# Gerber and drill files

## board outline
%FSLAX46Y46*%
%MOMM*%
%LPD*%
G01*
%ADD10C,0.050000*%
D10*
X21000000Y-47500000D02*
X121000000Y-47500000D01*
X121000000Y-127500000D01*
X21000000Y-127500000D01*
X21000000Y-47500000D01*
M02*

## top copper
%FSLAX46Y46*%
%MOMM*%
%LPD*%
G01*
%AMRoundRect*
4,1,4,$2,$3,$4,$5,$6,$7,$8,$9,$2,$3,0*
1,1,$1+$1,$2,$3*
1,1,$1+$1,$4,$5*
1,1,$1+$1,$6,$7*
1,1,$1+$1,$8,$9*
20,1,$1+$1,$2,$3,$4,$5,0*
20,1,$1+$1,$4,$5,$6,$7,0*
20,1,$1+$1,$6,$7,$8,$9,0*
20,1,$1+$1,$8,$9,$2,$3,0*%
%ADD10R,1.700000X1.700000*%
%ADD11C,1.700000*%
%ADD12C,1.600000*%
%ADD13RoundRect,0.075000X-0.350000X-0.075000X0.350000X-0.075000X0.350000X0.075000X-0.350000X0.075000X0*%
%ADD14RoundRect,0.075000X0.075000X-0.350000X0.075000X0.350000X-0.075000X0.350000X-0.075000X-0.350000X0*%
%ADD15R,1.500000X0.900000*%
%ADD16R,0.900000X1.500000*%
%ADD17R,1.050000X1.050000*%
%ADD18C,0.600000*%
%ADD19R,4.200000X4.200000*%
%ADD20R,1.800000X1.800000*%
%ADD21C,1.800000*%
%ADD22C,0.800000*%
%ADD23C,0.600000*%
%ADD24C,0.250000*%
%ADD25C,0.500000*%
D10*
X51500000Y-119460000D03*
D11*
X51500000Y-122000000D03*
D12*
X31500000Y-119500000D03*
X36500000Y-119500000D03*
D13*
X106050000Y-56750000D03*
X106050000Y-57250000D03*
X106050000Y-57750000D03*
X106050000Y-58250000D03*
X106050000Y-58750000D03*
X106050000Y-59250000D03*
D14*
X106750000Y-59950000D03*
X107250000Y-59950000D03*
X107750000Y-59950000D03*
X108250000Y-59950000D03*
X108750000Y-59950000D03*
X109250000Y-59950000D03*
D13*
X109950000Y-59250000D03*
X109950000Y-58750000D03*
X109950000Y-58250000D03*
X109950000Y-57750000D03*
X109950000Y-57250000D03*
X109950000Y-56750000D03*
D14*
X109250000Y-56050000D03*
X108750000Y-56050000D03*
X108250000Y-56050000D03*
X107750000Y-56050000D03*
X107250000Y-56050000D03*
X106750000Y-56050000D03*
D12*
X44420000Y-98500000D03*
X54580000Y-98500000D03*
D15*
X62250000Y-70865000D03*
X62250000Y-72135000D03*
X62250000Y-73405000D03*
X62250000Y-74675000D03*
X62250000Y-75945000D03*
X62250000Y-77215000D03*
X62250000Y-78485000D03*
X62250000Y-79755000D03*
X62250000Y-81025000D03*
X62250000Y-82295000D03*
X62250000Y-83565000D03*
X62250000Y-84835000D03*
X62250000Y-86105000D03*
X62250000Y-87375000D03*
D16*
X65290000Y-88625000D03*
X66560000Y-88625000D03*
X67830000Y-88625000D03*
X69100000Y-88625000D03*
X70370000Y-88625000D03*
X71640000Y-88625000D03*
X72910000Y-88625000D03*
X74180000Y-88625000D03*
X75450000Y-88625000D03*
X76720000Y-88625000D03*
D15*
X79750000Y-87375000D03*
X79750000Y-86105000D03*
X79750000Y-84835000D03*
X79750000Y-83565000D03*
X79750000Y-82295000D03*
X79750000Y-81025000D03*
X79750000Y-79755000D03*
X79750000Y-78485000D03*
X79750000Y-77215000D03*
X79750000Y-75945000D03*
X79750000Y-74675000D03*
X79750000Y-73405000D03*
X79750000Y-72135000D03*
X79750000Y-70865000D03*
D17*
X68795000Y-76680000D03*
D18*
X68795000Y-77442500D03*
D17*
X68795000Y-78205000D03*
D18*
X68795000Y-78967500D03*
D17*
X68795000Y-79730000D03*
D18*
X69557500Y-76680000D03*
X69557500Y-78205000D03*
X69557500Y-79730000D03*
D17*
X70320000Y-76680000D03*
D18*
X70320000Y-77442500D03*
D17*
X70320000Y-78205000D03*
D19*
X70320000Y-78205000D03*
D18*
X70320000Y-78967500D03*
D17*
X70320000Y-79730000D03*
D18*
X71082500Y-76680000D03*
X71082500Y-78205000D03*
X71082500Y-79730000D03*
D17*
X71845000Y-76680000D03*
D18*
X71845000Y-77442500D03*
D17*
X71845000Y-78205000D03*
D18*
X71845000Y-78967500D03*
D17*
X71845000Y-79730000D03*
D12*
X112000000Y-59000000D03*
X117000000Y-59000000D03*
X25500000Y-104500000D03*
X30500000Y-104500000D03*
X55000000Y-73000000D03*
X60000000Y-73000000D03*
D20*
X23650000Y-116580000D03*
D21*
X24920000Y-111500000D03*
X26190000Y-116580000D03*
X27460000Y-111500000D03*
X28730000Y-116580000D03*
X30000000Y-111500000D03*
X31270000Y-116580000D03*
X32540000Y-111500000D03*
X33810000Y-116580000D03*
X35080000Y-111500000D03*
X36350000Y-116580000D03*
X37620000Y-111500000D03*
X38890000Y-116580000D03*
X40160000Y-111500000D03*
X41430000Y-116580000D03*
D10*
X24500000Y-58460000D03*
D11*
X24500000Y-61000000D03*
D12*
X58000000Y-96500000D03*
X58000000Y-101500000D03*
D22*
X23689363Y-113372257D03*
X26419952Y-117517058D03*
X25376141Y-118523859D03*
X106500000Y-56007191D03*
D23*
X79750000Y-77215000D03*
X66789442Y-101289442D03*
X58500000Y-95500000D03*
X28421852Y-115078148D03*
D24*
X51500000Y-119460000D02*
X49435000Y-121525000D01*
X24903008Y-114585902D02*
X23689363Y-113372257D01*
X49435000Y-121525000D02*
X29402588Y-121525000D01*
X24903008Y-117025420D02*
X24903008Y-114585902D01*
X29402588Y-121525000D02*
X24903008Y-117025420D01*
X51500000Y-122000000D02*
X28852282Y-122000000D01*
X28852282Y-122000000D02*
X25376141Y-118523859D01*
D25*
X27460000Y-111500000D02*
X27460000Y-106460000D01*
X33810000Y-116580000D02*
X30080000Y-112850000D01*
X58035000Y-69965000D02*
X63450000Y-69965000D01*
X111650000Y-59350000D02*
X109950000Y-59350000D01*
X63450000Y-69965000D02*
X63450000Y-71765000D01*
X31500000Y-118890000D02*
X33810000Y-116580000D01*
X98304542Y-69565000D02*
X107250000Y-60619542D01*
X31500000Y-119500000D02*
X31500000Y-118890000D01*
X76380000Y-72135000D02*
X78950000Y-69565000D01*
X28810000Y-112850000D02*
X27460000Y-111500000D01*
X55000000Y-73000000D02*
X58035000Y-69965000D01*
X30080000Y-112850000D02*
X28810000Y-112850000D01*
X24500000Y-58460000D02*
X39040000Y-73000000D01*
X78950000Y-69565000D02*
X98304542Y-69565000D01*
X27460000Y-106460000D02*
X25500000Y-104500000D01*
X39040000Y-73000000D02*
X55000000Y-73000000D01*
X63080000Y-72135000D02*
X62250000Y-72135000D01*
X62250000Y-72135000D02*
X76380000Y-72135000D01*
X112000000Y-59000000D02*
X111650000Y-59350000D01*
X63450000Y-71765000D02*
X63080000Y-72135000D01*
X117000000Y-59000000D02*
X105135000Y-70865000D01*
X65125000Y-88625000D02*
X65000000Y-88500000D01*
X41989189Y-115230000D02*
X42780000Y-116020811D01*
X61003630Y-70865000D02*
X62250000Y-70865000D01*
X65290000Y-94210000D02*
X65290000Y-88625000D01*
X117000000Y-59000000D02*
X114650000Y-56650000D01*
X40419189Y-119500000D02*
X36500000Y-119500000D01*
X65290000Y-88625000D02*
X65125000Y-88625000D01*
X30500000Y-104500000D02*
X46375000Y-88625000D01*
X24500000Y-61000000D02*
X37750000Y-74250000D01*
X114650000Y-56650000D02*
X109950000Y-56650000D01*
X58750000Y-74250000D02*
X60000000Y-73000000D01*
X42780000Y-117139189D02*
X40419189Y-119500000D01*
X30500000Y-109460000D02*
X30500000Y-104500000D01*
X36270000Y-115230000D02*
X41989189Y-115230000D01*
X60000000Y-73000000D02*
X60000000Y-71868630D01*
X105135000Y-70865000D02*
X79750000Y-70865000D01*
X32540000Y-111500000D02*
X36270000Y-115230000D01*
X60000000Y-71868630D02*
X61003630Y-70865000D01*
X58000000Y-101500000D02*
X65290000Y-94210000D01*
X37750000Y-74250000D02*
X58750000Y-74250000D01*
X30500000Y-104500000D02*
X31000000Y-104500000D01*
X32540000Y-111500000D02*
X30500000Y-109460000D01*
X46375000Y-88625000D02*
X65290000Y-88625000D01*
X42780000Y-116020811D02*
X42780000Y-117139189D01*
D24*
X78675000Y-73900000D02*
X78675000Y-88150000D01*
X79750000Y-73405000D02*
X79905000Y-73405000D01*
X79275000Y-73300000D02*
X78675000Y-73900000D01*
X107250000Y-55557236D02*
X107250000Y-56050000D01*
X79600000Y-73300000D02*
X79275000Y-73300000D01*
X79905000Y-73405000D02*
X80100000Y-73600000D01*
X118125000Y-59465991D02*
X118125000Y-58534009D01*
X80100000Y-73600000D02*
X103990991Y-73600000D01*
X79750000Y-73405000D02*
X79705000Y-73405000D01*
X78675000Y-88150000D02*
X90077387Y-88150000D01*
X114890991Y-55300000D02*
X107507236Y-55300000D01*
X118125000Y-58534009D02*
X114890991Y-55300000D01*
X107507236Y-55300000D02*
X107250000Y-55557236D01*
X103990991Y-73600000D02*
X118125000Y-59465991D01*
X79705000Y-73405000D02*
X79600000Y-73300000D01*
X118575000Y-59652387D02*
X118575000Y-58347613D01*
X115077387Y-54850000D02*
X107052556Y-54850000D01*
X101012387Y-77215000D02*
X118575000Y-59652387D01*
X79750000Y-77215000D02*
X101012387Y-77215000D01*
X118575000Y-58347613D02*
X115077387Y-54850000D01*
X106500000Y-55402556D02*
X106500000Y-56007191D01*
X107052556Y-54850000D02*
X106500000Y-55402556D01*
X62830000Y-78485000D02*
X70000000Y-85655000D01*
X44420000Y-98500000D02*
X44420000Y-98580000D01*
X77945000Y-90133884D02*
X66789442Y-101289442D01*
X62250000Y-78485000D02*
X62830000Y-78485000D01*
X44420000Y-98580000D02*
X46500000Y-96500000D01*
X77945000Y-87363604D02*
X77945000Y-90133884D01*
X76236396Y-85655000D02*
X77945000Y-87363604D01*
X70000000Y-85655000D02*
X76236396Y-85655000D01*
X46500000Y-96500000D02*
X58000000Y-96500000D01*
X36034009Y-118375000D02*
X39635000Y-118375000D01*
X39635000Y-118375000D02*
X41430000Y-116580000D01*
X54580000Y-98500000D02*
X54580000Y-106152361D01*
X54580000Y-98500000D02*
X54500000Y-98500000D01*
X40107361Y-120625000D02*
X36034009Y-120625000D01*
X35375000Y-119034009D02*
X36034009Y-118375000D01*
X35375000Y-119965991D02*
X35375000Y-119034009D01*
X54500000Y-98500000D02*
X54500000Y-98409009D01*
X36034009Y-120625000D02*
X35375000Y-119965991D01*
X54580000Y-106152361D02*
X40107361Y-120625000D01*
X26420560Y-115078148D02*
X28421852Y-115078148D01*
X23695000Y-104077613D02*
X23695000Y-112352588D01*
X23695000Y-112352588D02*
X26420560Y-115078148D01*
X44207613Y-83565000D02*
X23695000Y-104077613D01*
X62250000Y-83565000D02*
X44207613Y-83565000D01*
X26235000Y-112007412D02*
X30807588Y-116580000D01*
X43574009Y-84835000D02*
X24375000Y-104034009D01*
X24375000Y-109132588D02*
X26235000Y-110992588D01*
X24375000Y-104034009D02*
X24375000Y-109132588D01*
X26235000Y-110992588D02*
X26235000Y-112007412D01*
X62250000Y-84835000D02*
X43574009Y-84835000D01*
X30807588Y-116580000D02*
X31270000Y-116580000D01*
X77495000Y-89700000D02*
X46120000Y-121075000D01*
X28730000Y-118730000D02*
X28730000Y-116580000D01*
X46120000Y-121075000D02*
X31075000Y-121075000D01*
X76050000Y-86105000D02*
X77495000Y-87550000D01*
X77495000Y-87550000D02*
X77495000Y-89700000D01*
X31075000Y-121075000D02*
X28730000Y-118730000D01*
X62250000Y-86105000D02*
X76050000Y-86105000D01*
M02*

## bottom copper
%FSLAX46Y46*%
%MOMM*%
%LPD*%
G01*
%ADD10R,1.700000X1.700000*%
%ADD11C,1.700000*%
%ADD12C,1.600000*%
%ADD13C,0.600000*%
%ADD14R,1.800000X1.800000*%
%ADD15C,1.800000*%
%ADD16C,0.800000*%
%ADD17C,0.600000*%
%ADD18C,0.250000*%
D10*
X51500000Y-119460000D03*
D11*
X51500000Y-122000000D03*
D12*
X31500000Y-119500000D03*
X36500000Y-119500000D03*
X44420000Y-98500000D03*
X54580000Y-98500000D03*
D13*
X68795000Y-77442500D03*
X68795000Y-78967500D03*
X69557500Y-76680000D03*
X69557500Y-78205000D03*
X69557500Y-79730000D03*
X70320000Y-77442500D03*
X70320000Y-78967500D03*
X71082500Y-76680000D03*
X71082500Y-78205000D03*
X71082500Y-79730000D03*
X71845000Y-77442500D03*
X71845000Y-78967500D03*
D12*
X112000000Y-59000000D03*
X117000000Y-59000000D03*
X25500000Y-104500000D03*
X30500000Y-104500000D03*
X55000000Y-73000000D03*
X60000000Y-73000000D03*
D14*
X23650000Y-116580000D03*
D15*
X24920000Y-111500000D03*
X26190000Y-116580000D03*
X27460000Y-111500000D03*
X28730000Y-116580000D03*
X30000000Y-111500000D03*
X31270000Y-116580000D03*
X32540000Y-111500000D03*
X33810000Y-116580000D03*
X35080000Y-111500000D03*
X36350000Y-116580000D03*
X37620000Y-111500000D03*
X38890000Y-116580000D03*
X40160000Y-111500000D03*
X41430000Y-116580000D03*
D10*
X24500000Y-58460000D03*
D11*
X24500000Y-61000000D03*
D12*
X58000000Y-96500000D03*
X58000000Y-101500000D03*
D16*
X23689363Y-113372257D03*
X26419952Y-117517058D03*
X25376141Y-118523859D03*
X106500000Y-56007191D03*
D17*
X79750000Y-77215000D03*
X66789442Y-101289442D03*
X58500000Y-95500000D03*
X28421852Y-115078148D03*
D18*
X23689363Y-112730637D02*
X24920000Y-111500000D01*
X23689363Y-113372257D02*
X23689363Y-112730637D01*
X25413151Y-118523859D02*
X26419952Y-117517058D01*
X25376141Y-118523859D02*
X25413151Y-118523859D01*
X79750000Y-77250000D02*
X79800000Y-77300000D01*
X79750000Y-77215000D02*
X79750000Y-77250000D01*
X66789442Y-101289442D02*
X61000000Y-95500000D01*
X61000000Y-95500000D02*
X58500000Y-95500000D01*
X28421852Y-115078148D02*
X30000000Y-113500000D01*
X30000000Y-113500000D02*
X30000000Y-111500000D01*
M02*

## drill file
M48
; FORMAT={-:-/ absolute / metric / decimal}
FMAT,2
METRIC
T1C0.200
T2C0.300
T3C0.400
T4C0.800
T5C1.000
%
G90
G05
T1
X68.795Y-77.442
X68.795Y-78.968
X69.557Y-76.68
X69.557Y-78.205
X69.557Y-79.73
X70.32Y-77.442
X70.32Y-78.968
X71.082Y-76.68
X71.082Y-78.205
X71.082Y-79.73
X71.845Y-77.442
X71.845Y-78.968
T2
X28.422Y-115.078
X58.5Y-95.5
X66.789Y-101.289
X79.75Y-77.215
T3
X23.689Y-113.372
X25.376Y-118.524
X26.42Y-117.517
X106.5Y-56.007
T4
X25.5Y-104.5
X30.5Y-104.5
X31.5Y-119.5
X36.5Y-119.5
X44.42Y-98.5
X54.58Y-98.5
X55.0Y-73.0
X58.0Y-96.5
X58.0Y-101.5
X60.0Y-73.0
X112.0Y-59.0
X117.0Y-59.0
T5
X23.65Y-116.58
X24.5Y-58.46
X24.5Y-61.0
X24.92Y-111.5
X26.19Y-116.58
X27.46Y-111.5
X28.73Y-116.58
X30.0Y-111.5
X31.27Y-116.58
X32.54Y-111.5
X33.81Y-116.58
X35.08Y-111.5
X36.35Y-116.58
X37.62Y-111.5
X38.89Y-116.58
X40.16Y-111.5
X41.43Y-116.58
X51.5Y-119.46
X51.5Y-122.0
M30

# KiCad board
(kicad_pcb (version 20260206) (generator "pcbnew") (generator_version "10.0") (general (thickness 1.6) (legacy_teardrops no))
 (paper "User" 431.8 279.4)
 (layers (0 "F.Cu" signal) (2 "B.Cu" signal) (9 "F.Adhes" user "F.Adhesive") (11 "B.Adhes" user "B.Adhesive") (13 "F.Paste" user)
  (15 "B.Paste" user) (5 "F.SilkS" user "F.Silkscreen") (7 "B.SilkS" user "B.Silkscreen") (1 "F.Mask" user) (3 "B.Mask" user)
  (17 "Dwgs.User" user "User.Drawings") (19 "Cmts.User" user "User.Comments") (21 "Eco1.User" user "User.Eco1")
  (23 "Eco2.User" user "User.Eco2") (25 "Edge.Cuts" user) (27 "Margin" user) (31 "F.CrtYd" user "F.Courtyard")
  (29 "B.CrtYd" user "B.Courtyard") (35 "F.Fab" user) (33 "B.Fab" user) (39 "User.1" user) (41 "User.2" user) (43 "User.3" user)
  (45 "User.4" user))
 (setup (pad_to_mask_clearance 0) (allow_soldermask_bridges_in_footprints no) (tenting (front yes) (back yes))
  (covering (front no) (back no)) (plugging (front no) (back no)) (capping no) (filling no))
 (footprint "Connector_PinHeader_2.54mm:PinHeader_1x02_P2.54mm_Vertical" (layer "F.Cu") (at 51.5 119.46)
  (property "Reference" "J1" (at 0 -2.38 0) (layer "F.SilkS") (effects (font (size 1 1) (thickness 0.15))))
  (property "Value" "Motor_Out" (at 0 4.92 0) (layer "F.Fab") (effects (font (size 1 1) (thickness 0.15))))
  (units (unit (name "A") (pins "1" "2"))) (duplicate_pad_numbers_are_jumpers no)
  (pad "1" thru_hole rect (at 0 0) (size 1.7 1.7) (drill 1) (layers "*.Cu" "*.Mask") (remove_unused_layers no) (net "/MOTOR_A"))
  (pad "2" thru_hole circle (at 0 2.54) (size 1.7 1.7) (drill 1) (layers "*.Cu" "*.Mask") (remove_unused_layers no) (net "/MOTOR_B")))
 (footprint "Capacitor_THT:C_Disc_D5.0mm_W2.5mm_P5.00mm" (layer "F.Cu") (at 31.5 119.5)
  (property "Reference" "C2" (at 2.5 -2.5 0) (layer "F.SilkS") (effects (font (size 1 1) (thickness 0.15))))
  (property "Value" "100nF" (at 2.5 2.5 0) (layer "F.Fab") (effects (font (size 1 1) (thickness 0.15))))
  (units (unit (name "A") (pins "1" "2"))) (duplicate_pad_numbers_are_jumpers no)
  (pad "1" thru_hole circle (at 0 0) (size 1.6 1.6) (drill 0.8) (layers "*.Cu" "*.Mask") (remove_unused_layers no) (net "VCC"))
  (pad "2" thru_hole circle (at 5 0) (size 1.6 1.6) (drill 0.8) (layers "*.Cu" "*.Mask") (remove_unused_layers no) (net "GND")))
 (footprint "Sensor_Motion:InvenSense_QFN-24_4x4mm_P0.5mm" (layer "F.Cu") (at 108 58)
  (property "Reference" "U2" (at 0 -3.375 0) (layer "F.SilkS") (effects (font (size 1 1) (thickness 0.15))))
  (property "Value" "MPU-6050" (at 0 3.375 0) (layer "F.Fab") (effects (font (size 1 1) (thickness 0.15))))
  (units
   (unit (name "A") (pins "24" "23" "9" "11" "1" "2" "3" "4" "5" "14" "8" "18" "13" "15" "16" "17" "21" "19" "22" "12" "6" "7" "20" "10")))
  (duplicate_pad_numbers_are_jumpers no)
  (pad "1" smd roundrect (at -1.95 -1.25) (size 0.85 0.3) (layers "F.Cu" "F.Mask" "F.Paste") (roundrect_rratio 0.25)
   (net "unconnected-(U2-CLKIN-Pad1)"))
  (pad "2" smd roundrect (at -1.95 -0.75) (size 0.85 0.3) (layers "F.Cu" "F.Mask" "F.Paste") (roundrect_rratio 0.25)
   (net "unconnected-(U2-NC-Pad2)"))
  (pad "3" smd roundrect (at -1.95 -0.25) (size 0.85 0.3) (layers "F.Cu" "F.Mask" "F.Paste") (roundrect_rratio 0.25)
   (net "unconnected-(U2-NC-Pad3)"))
  (pad "4" smd roundrect (at -1.95 0.25) (size 0.85 0.3) (layers "F.Cu" "F.Mask" "F.Paste") (roundrect_rratio 0.25)
   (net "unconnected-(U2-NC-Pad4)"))
  (pad "5" smd roundrect (at -1.95 0.75) (size 0.85 0.3) (layers "F.Cu" "F.Mask" "F.Paste") (roundrect_rratio 0.25)
   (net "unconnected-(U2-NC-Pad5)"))
  (pad "6" smd roundrect (at -1.95 1.25) (size 0.85 0.3) (layers "F.Cu" "F.Mask" "F.Paste") (roundrect_rratio 0.25)
   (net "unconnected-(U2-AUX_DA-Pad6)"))
  (pad "7" smd roundrect (at -1.25 1.95 90) (size 0.85 0.3) (layers "F.Cu" "F.Mask" "F.Paste") (roundrect_rratio 0.25)
   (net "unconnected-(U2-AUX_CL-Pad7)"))
  (pad "8" smd roundrect (at -0.75 1.95 90) (size 0.85 0.3) (layers "F.Cu" "F.Mask" "F.Paste") (roundrect_rratio 0.25) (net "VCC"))
  (pad "9" smd roundrect (at -0.25 1.95 90) (size 0.85 0.3) (layers "F.Cu" "F.Mask" "F.Paste") (roundrect_rratio 0.25)
   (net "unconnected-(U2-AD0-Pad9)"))
  (pad "10" smd roundrect (at 0.25 1.95 90) (size 0.85 0.3) (layers "F.Cu" "F.Mask" "F.Paste") (roundrect_rratio 0.25)
   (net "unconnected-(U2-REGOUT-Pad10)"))
  (pad "11" smd roundrect (at 0.75 1.95 90) (size 0.85 0.3) (layers "F.Cu" "F.Mask" "F.Paste") (roundrect_rratio 0.25)
   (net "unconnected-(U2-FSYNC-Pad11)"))
  (pad "12" smd roundrect (at 1.25 1.95 90) (size 0.85 0.3) (layers "F.Cu" "F.Mask" "F.Paste") (roundrect_rratio 0.25)
   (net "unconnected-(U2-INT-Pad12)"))
  (pad "13" smd roundrect (at 1.95 1.25) (size 0.85 0.3) (layers "F.Cu" "F.Mask" "F.Paste") (roundrect_rratio 0.25) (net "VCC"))
  (pad "14" smd roundrect (at 1.95 0.75) (size 0.85 0.3) (layers "F.Cu" "F.Mask" "F.Paste") (roundrect_rratio 0.25)
   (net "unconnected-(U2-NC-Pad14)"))
  (pad "15" smd roundrect (at 1.95 0.25) (size 0.85 0.3) (layers "F.Cu" "F.Mask" "F.Paste") (roundrect_rratio 0.25)
   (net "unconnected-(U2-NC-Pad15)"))
  (pad "16" smd roundrect (at 1.95 -0.25) (size 0.85 0.3) (layers "F.Cu" "F.Mask" "F.Paste") (roundrect_rratio 0.25)
   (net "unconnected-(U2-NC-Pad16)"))
  (pad "17" smd roundrect (at 1.95 -0.75) (size 0.85 0.3) (layers "F.Cu" "F.Mask" "F.Paste") (roundrect_rratio 0.25)
   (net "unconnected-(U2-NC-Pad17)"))
  (pad "18" smd roundrect (at 1.95 -1.25) (size 0.85 0.3) (layers "F.Cu" "F.Mask" "F.Paste") (roundrect_rratio 0.25) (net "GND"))
  (pad "19" smd roundrect (at 1.25 -1.95 90) (size 0.85 0.3) (layers "F.Cu" "F.Mask" "F.Paste") (roundrect_rratio 0.25)
   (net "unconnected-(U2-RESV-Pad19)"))
  (pad "20" smd roundrect (at 0.75 -1.95 90) (size 0.85 0.3) (layers "F.Cu" "F.Mask" "F.Paste") (roundrect_rratio 0.25)
   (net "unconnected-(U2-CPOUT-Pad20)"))
  (pad "21" smd roundrect (at 0.25 -1.95 90) (size 0.85 0.3) (layers "F.Cu" "F.Mask" "F.Paste") (roundrect_rratio 0.25)
   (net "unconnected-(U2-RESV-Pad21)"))
  (pad "22" smd roundrect (at -0.25 -1.95 90) (size 0.85 0.3) (layers "F.Cu" "F.Mask" "F.Paste") (roundrect_rratio 0.25)
   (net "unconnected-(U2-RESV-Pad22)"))
  (pad "23" smd roundrect (at -0.75 -1.95 90) (size 0.85 0.3) (layers "F.Cu" "F.Mask" "F.Paste") (roundrect_rratio 0.25) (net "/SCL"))
  (pad "24" smd roundrect (at -1.25 -1.95 90) (size 0.85 0.3) (layers "F.Cu" "F.Mask" "F.Paste") (roundrect_rratio 0.25) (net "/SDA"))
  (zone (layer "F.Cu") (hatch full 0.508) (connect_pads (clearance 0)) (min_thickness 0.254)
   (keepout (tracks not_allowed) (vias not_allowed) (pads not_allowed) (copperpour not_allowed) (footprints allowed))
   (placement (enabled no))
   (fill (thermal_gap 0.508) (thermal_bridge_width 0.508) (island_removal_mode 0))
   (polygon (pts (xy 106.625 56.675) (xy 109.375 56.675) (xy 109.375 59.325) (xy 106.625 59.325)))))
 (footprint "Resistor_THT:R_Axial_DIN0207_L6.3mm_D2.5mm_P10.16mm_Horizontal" (layer "F.Cu") (at 44.42 98.5)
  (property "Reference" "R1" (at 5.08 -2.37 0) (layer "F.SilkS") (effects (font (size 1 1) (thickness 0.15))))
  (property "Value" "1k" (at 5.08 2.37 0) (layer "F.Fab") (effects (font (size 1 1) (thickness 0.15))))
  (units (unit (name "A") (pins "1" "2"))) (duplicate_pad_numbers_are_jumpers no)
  (pad "1" thru_hole circle (at 0 0) (size 1.6 1.6) (drill 0.8) (layers "*.Cu" "*.Mask") (remove_unused_layers no) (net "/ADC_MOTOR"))
  (pad "2" thru_hole circle (at 10.16 0) (size 1.6 1.6) (drill 0.8) (layers "*.Cu" "*.Mask") (remove_unused_layers no) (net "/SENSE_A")))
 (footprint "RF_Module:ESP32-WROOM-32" (layer "F.Cu") (at 71 79.115)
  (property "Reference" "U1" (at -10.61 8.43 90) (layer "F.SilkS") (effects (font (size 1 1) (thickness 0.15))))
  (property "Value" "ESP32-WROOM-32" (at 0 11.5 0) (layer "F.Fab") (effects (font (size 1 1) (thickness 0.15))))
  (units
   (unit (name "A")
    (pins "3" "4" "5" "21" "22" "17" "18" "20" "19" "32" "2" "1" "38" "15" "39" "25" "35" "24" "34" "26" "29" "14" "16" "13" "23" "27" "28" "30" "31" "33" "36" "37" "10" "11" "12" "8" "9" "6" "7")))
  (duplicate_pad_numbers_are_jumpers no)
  (pad "1" smd rect (at -8.75 -8.25) (size 1.5 0.9) (layers "F.Cu" "F.Mask" "F.Paste") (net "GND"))
  (pad "2" smd rect (at -8.75 -6.98) (size 1.5 0.9) (layers "F.Cu" "F.Mask" "F.Paste") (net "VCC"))
  (pad "3" smd rect (at -8.75 -5.71) (size 1.5 0.9) (layers "F.Cu" "F.Mask" "F.Paste") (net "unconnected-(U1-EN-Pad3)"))
  (pad "4" smd rect (at -8.75 -4.44) (size 1.5 0.9) (layers "F.Cu" "F.Mask" "F.Paste") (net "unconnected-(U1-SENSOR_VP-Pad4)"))
  (pad "5" smd rect (at -8.75 -3.17) (size 1.5 0.9) (layers "F.Cu" "F.Mask" "F.Paste") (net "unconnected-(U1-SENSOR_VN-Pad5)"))
  (pad "6" smd rect (at -8.75 -1.9) (size 1.5 0.9) (layers "F.Cu" "F.Mask" "F.Paste") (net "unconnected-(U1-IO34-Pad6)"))
  (pad "7" smd rect (at -8.75 -0.63) (size 1.5 0.9) (layers "F.Cu" "F.Mask" "F.Paste") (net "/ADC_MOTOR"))
  (pad "8" smd rect (at -8.75 0.64) (size 1.5 0.9) (layers "F.Cu" "F.Mask" "F.Paste") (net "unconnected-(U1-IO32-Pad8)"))
  (pad "9" smd rect (at -8.75 1.91) (size 1.5 0.9) (layers "F.Cu" "F.Mask" "F.Paste") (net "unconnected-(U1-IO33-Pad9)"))
  (pad "10" smd rect (at -8.75 3.18) (size 1.5 0.9) (layers "F.Cu" "F.Mask" "F.Paste") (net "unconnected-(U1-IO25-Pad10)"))
  (pad "11" smd rect (at -8.75 4.45) (size 1.5 0.9) (layers "F.Cu" "F.Mask" "F.Paste") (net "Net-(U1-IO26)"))
  (pad "12" smd rect (at -8.75 5.72) (size 1.5 0.9) (layers "F.Cu" "F.Mask" "F.Paste") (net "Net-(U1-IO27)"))
  (pad "13" smd rect (at -8.75 6.99) (size 1.5 0.9) (layers "F.Cu" "F.Mask" "F.Paste") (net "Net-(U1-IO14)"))
  (pad "14" smd rect (at -8.75 8.26) (size 1.5 0.9) (layers "F.Cu" "F.Mask" "F.Paste") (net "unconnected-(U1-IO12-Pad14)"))
  (pad "15" smd rect (at -5.71 9.51 90) (size 1.5 0.9) (layers "F.Cu" "F.Mask" "F.Paste") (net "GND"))
  (pad "16" smd rect (at -4.44 9.51 90) (size 1.5 0.9) (layers "F.Cu" "F.Mask" "F.Paste") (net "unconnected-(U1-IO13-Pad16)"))
  (pad "17" smd rect (at -3.17 9.51 90) (size 1.5 0.9) (layers "F.Cu" "F.Mask" "F.Paste") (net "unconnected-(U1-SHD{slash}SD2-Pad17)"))
  (pad "18" smd rect (at -1.9 9.51 90) (size 1.5 0.9) (layers "F.Cu" "F.Mask" "F.Paste") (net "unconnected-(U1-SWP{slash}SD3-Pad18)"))
  (pad "19" smd rect (at -0.63 9.51 90) (size 1.5 0.9) (layers "F.Cu" "F.Mask" "F.Paste") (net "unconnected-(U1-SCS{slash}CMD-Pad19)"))
  (pad "20" smd rect (at 0.64 9.51 90) (size 1.5 0.9) (layers "F.Cu" "F.Mask" "F.Paste") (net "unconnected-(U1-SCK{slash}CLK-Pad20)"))
  (pad "21" smd rect (at 1.91 9.51 90) (size 1.5 0.9) (layers "F.Cu" "F.Mask" "F.Paste") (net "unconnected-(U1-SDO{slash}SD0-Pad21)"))
  (pad "22" smd rect (at 3.18 9.51 90) (size 1.5 0.9) (layers "F.Cu" "F.Mask" "F.Paste") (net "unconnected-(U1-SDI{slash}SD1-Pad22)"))
  (pad "23" smd rect (at 4.45 9.51 90) (size 1.5 0.9) (layers "F.Cu" "F.Mask" "F.Paste") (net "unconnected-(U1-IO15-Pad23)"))
  (pad "24" smd rect (at 5.72 9.51 90) (size 1.5 0.9) (layers "F.Cu" "F.Mask" "F.Paste") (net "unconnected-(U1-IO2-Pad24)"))
  (pad "25" smd rect (at 8.75 8.26) (size 1.5 0.9) (layers "F.Cu" "F.Mask" "F.Paste") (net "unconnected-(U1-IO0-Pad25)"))
  (pad "26" smd rect (at 8.75 6.99) (size 1.5 0.9) (layers "F.Cu" "F.Mask" "F.Paste") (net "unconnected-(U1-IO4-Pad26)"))
  (pad "27" smd rect (at 8.75 5.72) (size 1.5 0.9) (layers "F.Cu" "F.Mask" "F.Paste") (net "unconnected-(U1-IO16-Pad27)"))
  (pad "28" smd rect (at 8.75 4.45) (size 1.5 0.9) (layers "F.Cu" "F.Mask" "F.Paste") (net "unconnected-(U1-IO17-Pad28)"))
  (pad "29" smd rect (at 8.75 3.18) (size 1.5 0.9) (layers "F.Cu" "F.Mask" "F.Paste") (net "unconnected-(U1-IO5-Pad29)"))
  (pad "30" smd rect (at 8.75 1.91) (size 1.5 0.9) (layers "F.Cu" "F.Mask" "F.Paste") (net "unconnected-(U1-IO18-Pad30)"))
  (pad "31" smd rect (at 8.75 0.64) (size 1.5 0.9) (layers "F.Cu" "F.Mask" "F.Paste") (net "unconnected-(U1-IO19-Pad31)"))
  (pad "32" smd rect (at 8.75 -0.63) (size 1.5 0.9) (layers "F.Cu" "F.Mask" "F.Paste") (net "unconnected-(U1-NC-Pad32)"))
  (pad "33" smd rect (at 8.75 -1.9) (size 1.5 0.9) (layers "F.Cu" "F.Mask" "F.Paste") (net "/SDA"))
  (pad "34" smd rect (at 8.75 -3.17) (size 1.5 0.9) (layers "F.Cu" "F.Mask" "F.Paste") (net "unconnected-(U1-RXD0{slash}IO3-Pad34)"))
  (pad "35" smd rect (at 8.75 -4.44) (size 1.5 0.9) (layers "F.Cu" "F.Mask" "F.Paste") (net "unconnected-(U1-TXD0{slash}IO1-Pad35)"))
  (pad "36" smd rect (at 8.75 -5.71) (size 1.5 0.9) (layers "F.Cu" "F.Mask" "F.Paste") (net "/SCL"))
  (pad "37" smd rect (at 8.75 -6.98) (size 1.5 0.9) (layers "F.Cu" "F.Mask" "F.Paste") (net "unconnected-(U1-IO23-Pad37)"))
  (pad "38" smd rect (at 8.75 -8.25) (size 1.5 0.9) (layers "F.Cu" "F.Mask" "F.Paste") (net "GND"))
  (pad "39" smd rect (at -2.205 -2.435) (size 1.05 1.05) (layers "F.Cu" "F.Paste") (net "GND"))
  (pad "39" thru_hole circle (at -2.205 -1.6725) (size 0.6 0.6) (drill 0.2) (layers "*.Cu" "F.Mask") (remove_unused_layers no) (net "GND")
   (zone_connect 2))
  (pad "39" smd rect (at -2.205 -0.91) (size 1.05 1.05) (layers "F.Cu" "F.Paste") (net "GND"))
  (pad "39" thru_hole circle (at -2.205 -0.1475) (size 0.6 0.6) (drill 0.2) (layers "*.Cu" "F.Mask") (remove_unused_layers no) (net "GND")
   (zone_connect 2))
  (pad "39" smd rect (at -2.205 0.615) (size 1.05 1.05) (layers "F.Cu" "F.Paste") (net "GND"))
  (pad "39" thru_hole circle (at -1.4425 -2.435) (size 0.6 0.6) (drill 0.2) (layers "*.Cu" "F.Mask") (remove_unused_layers no) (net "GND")
   (zone_connect 2))
  (pad "39" thru_hole circle (at -1.4425 -0.91) (size 0.6 0.6) (drill 0.2) (layers "*.Cu" "F.Mask") (remove_unused_layers no) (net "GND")
   (zone_connect 2))
  (pad "39" thru_hole circle (at -1.4425 0.615) (size 0.6 0.6) (drill 0.2) (layers "*.Cu" "F.Mask") (remove_unused_layers no) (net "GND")
   (zone_connect 2))
  (pad "39" smd rect (at -0.68 -2.435) (size 1.05 1.05) (layers "F.Cu" "F.Paste") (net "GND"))
  (pad "39" thru_hole circle (at -0.68 -1.6725) (size 0.6 0.6) (drill 0.2) (layers "*.Cu" "F.Mask") (remove_unused_layers no) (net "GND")
   (zone_connect 2))
  (pad "39" smd rect (at -0.68 -0.91) (size 1.05 1.05) (layers "F.Cu" "F.Paste") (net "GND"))
  (pad "39" smd rect (at -0.68 -0.91) (size 4.2 4.2) (layers "F.Cu" "F.Mask") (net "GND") (zone_connect 2))
  (pad "39" thru_hole circle (at -0.68 -0.1475) (size 0.6 0.6) (drill 0.2) (layers "*.Cu" "F.Mask") (remove_unused_layers no) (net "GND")
   (zone_connect 2))
  (pad "39" smd rect (at -0.68 0.615) (size 1.05 1.05) (layers "F.Cu" "F.Paste") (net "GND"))
  (pad "39" thru_hole circle (at 0.0825 -2.435) (size 0.6 0.6) (drill 0.2) (layers "*.Cu" "F.Mask") (remove_unused_layers no) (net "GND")
   (zone_connect 2))
  (pad "39" thru_hole circle (at 0.0825 -0.91) (size 0.6 0.6) (drill 0.2) (layers "*.Cu" "F.Mask") (remove_unused_layers no) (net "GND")
   (zone_connect 2))
  (pad "39" thru_hole circle (at 0.0825 0.615) (size 0.6 0.6) (drill 0.2) (layers "*.Cu" "F.Mask") (remove_unused_layers no) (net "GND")
   (zone_connect 2))
  (pad "39" smd rect (at 0.845 -2.435) (size 1.05 1.05) (layers "F.Cu" "F.Paste") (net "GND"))
  (pad "39" thru_hole circle (at 0.845 -1.6725) (size 0.6 0.6) (drill 0.2) (layers "*.Cu" "F.Mask") (remove_unused_layers no) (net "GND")
   (zone_connect 2))
  (pad "39" smd rect (at 0.845 -0.91) (size 1.05 1.05) (layers "F.Cu" "F.Paste") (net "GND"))
  (pad "39" thru_hole circle (at 0.845 -0.1475) (size 0.6 0.6) (drill 0.2) (layers "*.Cu" "F.Mask") (remove_unused_layers no) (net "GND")
   (zone_connect 2))
  (pad "39" smd rect (at 0.845 0.615) (size 1.05 1.05) (layers "F.Cu" "F.Paste") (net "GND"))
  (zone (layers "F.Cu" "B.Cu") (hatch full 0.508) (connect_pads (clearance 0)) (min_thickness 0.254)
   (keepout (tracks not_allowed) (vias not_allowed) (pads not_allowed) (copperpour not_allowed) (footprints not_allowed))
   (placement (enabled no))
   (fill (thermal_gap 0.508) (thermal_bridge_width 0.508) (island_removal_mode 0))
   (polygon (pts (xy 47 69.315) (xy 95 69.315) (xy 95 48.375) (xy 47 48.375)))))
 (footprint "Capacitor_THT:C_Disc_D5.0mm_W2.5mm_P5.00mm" (layer "F.Cu") (at 112 59)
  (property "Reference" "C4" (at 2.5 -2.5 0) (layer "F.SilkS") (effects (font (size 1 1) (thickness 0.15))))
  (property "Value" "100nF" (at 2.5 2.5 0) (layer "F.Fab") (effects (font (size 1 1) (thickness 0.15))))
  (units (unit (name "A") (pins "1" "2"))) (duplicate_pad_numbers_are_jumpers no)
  (pad "1" thru_hole circle (at 0 0) (size 1.6 1.6) (drill 0.8) (layers "*.Cu" "*.Mask") (remove_unused_layers no) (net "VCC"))
  (pad "2" thru_hole circle (at 5 0) (size 1.6 1.6) (drill 0.8) (layers "*.Cu" "*.Mask") (remove_unused_layers no) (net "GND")))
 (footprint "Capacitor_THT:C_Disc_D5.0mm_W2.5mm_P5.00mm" (layer "F.Cu") (at 25.5 104.5)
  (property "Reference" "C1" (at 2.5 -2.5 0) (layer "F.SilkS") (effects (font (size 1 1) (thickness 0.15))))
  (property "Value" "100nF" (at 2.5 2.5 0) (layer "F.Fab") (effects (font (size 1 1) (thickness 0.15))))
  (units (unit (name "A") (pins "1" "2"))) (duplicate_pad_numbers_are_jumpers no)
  (pad "1" thru_hole circle (at 0 0) (size 1.6 1.6) (drill 0.8) (layers "*.Cu" "*.Mask") (remove_unused_layers no) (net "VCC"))
  (pad "2" thru_hole circle (at 5 0) (size 1.6 1.6) (drill 0.8) (layers "*.Cu" "*.Mask") (remove_unused_layers no) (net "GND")))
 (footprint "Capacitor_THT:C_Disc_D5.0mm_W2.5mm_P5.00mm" (layer "F.Cu") (at 55 73)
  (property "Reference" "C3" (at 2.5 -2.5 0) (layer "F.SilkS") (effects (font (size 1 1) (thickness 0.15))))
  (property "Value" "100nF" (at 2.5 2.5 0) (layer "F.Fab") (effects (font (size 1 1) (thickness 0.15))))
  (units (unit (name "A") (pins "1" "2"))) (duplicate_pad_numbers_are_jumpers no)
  (pad "1" thru_hole circle (at 0 0) (size 1.6 1.6) (drill 0.8) (layers "*.Cu" "*.Mask") (remove_unused_layers no) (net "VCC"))
  (pad "2" thru_hole circle (at 5 0) (size 1.6 1.6) (drill 0.8) (layers "*.Cu" "*.Mask") (remove_unused_layers no) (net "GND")))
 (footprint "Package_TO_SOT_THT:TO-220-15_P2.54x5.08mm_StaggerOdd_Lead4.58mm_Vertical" (layer "F.Cu") (at 23.65 116.58)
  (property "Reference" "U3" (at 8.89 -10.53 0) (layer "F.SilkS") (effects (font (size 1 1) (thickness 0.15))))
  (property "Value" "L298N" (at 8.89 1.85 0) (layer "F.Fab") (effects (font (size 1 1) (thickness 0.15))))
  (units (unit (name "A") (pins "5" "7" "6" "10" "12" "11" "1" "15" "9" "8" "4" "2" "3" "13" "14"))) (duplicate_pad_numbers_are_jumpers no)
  (pad "1" thru_hole rect (at 0 0) (size 1.8 1.8) (drill 1) (layers "*.Cu" "*.Mask") (remove_unused_layers no)
   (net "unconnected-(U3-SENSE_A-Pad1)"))
  (pad "2" thru_hole circle (at 1.27 -5.08) (size 1.8 1.8) (drill 1) (layers "*.Cu" "*.Mask") (remove_unused_layers no) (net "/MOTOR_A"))
  (pad "3" thru_hole circle (at 2.54 0) (size 1.8 1.8) (drill 1) (layers "*.Cu" "*.Mask") (remove_unused_layers no) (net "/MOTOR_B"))
  (pad "4" thru_hole circle (at 3.81 -5.08) (size 1.8 1.8) (drill 1) (layers "*.Cu" "*.Mask") (remove_unused_layers no) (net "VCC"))
  (pad "5" thru_hole circle (at 5.08 0) (size 1.8 1.8) (drill 1) (layers "*.Cu" "*.Mask") (remove_unused_layers no) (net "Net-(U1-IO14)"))
  (pad "6" thru_hole circle (at 6.35 -5.08) (size 1.8 1.8) (drill 1) (layers "*.Cu" "*.Mask") (remove_unused_layers no)
   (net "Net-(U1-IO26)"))
  (pad "7" thru_hole circle (at 7.62 0) (size 1.8 1.8) (drill 1) (layers "*.Cu" "*.Mask") (remove_unused_layers no) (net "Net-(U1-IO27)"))
  (pad "8" thru_hole circle (at 8.89 -5.08) (size 1.8 1.8) (drill 1) (layers "*.Cu" "*.Mask") (remove_unused_layers no) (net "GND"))
  (pad "9" thru_hole circle (at 10.16 0) (size 1.8 1.8) (drill 1) (layers "*.Cu" "*.Mask") (remove_unused_layers no) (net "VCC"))
  (pad "10" thru_hole circle (at 11.43 -5.08) (size 1.8 1.8) (drill 1) (layers "*.Cu" "*.Mask") (remove_unused_layers no)
   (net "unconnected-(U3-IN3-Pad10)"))
  (pad "11" thru_hole circle (at 12.7 0) (size 1.8 1.8) (drill 1) (layers "*.Cu" "*.Mask") (remove_unused_layers no)
   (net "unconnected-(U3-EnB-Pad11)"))
  (pad "12" thru_hole circle (at 13.97 -5.08) (size 1.8 1.8) (drill 1) (layers "*.Cu" "*.Mask") (remove_unused_layers no)
   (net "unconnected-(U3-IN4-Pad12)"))
  (pad "13" thru_hole circle (at 15.24 0) (size 1.8 1.8) (drill 1) (layers "*.Cu" "*.Mask") (remove_unused_layers no)
   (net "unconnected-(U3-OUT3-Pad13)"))
  (pad "14" thru_hole circle (at 16.51 -5.08) (size 1.8 1.8) (drill 1) (layers "*.Cu" "*.Mask") (remove_unused_layers no)
   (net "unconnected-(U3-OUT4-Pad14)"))
  (pad "15" thru_hole circle (at 17.78 0) (size 1.8 1.8) (drill 1) (layers "*.Cu" "*.Mask") (remove_unused_layers no) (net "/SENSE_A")))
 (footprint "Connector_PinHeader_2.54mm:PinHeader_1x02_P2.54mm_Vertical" (layer "F.Cu") (at 24.5 58.46)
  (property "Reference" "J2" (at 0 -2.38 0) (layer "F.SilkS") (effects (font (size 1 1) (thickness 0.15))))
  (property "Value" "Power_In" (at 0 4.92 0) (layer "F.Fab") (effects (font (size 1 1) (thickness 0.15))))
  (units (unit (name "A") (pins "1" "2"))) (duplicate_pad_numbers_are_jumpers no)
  (pad "1" thru_hole rect (at 0 0) (size 1.7 1.7) (drill 1) (layers "*.Cu" "*.Mask") (remove_unused_layers no) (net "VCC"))
  (pad "2" thru_hole circle (at 0 2.54) (size 1.7 1.7) (drill 1) (layers "*.Cu" "*.Mask") (remove_unused_layers no) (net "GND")))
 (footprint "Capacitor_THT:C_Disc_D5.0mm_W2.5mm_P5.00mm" (layer "F.Cu") (at 58 96.5 -90)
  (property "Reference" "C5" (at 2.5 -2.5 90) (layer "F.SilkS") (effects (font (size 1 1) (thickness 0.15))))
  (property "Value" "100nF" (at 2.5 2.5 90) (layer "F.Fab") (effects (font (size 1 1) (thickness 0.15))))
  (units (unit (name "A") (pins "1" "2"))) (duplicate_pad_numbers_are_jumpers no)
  (pad "1" thru_hole circle (at 0 0 270) (size 1.6 1.6) (drill 0.8) (layers "*.Cu" "*.Mask") (remove_unused_layers no) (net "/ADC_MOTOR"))
  (pad "2" thru_hole circle (at 5 0 270) (size 1.6 1.6) (drill 0.8) (layers "*.Cu" "*.Mask") (remove_unused_layers no) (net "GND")))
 (gr_rect (start 21 47.5) (end 121 127.5) (stroke (width 0.05) (type solid)) (fill no) (layer "Edge.Cuts"))
 (segment (start 51.5 119.46) (end 49.435 121.525) (width 0.25) (layer "F.Cu") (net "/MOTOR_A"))
 (segment (start 24.903008 114.585902) (end 23.689363 113.372257) (width 0.25) (layer "F.Cu") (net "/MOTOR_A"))
 (segment (start 49.435 121.525) (end 29.402588 121.525) (width 0.25) (layer "F.Cu") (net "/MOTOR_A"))
 (segment (start 24.903008 117.02542) (end 24.903008 114.585902) (width 0.25) (layer "F.Cu") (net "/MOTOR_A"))
 (segment (start 29.402588 121.525) (end 24.903008 117.02542) (width 0.25) (layer "F.Cu") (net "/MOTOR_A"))
 (via (at 23.689363 113.372257) (size 0.8) (drill 0.4) (layers "F.Cu" "B.Cu") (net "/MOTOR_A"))
 (segment (start 23.689363 112.730637) (end 24.92 111.5) (width 0.25) (layer "B.Cu") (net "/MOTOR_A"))
 (segment (start 23.689363 113.372257) (end 23.689363 112.730637) (width 0.25) (layer "B.Cu") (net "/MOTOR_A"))
 (segment (start 51.5 122) (end 28.852282 122) (width 0.25) (layer "F.Cu") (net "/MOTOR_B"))
 (segment (start 28.852282 122) (end 25.376141 118.523859) (width 0.25) (layer "F.Cu") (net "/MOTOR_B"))
 (via (at 26.419952 117.517058) (size 0.8) (drill 0.4) (layers "F.Cu" "B.Cu") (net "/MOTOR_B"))
 (via (at 25.376141 118.523859) (size 0.8) (drill 0.4) (layers "F.Cu" "B.Cu") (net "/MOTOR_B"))
 (segment (start 25.413151 118.523859) (end 26.419952 117.517058) (width 0.25) (layer "B.Cu") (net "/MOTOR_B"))
 (segment (start 25.376141 118.523859) (end 25.413151 118.523859) (width 0.25) (layer "B.Cu") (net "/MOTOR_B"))
 (segment (start 27.46 111.5) (end 27.46 106.46) (width 0.5) (layer "F.Cu") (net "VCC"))
 (segment (start 33.81 116.58) (end 30.08 112.85) (width 0.5) (layer "F.Cu") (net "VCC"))
 (segment (start 58.035 69.965) (end 63.45 69.965) (width 0.5) (layer "F.Cu") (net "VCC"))
 (segment (start 111.65 59.35) (end 109.95 59.35) (width 0.5) (layer "F.Cu") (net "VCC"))
 (segment (start 63.45 69.965) (end 63.45 71.765) (width 0.5) (layer "F.Cu") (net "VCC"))
 (segment (start 31.5 118.89) (end 33.81 116.58) (width 0.5) (layer "F.Cu") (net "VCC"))
 (segment (start 98.304542 69.565) (end 107.25 60.619542) (width 0.5) (layer "F.Cu") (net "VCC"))
 (segment (start 31.5 119.5) (end 31.5 118.89) (width 0.5) (layer "F.Cu") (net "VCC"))
 (segment (start 76.38 72.135) (end 78.95 69.565) (width 0.5) (layer "F.Cu") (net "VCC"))
 (segment (start 28.81 112.85) (end 27.46 111.5) (width 0.5) (layer "F.Cu") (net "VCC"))
 (segment (start 55 73) (end 58.035 69.965) (width 0.5) (layer "F.Cu") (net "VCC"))
 (segment (start 30.08 112.85) (end 28.81 112.85) (width 0.5) (layer "F.Cu") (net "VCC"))
 (segment (start 24.5 58.46) (end 39.04 73) (width 0.5) (layer "F.Cu") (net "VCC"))
 (segment (start 78.95 69.565) (end 98.304542 69.565) (width 0.5) (layer "F.Cu") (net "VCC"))
 (segment (start 27.46 106.46) (end 25.5 104.5) (width 0.5) (layer "F.Cu") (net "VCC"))
 (segment (start 39.04 73) (end 55 73) (width 0.5) (layer "F.Cu") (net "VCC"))
 (segment (start 63.08 72.135) (end 62.25 72.135) (width 0.5) (layer "F.Cu") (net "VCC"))
 (segment (start 62.25 72.135) (end 76.38 72.135) (width 0.5) (layer "F.Cu") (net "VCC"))
 (segment (start 112 59) (end 111.65 59.35) (width 0.5) (layer "F.Cu") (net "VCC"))
 (segment (start 63.45 71.765) (end 63.08 72.135) (width 0.5) (layer "F.Cu") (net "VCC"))
 (segment (start 117 59) (end 105.135 70.865) (width 0.5) (layer "F.Cu") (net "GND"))
 (segment (start 65.125 88.625) (end 65 88.5) (width 0.5) (layer "F.Cu") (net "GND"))
 (segment (start 41.989189 115.23) (end 42.78 116.020811) (width 0.5) (layer "F.Cu") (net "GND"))
 (segment (start 61.00363 70.865) (end 62.25 70.865) (width 0.5) (layer "F.Cu") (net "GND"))
 (segment (start 65.29 94.21) (end 65.29 88.625) (width 0.5) (layer "F.Cu") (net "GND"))
 (segment (start 117 59) (end 114.65 56.65) (width 0.5) (layer "F.Cu") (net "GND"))
 (segment (start 40.419189 119.5) (end 36.5 119.5) (width 0.5) (layer "F.Cu") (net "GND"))
 (segment (start 65.29 88.625) (end 65.125 88.625) (width 0.5) (layer "F.Cu") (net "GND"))
 (segment (start 30.5 104.5) (end 46.375 88.625) (width 0.5) (layer "F.Cu") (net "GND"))
 (segment (start 24.5 61) (end 37.75 74.25) (width 0.5) (layer "F.Cu") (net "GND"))
 (segment (start 114.65 56.65) (end 109.95 56.65) (width 0.5) (layer "F.Cu") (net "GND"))
 (segment (start 58.75 74.25) (end 60 73) (width 0.5) (layer "F.Cu") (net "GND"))
 (segment (start 42.78 117.139189) (end 40.419189 119.5) (width 0.5) (layer "F.Cu") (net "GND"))
 (segment (start 30.5 109.46) (end 30.5 104.5) (width 0.5) (layer "F.Cu") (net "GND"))
 (segment (start 36.27 115.23) (end 41.989189 115.23) (width 0.5) (layer "F.Cu") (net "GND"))
 (segment (start 60 73) (end 60 71.86863) (width 0.5) (layer "F.Cu") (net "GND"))
 (segment (start 105.135 70.865) (end 79.75 70.865) (width 0.5) (layer "F.Cu") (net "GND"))
 (segment (start 32.54 111.5) (end 36.27 115.23) (width 0.5) (layer "F.Cu") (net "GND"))
 (segment (start 60 71.86863) (end 61.00363 70.865) (width 0.5) (layer "F.Cu") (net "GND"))
 (segment (start 58 101.5) (end 65.29 94.21) (width 0.5) (layer "F.Cu") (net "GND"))
 (segment (start 37.75 74.25) (end 58.75 74.25) (width 0.5) (layer "F.Cu") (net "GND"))
 (segment (start 30.5 104.5) (end 31 104.5) (width 0.5) (layer "F.Cu") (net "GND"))
 (segment (start 32.54 111.5) (end 30.5 109.46) (width 0.5) (layer "F.Cu") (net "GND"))
 (segment (start 46.375 88.625) (end 65.29 88.625) (width 0.5) (layer "F.Cu") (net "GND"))
 (segment (start 42.78 116.020811) (end 42.78 117.139189) (width 0.5) (layer "F.Cu") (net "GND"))
 (segment (start 78.675 73.9) (end 78.675 88.15) (width 0.25) (layer "F.Cu") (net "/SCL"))
 (segment (start 79.75 73.405) (end 79.905 73.405) (width 0.25) (layer "F.Cu") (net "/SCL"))
 (segment (start 79.275 73.3) (end 78.675 73.9) (width 0.25) (layer "F.Cu") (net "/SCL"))
 (segment (start 107.25 55.557236) (end 107.25 56.05) (width 0.25) (layer "F.Cu") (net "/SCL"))
 (segment (start 79.6 73.3) (end 79.275 73.3) (width 0.25) (layer "F.Cu") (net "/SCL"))
 (segment (start 79.905 73.405) (end 80.1 73.6) (width 0.25) (layer "F.Cu") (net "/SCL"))
 (segment (start 118.125 59.465991) (end 118.125 58.534009) (width 0.25) (layer "F.Cu") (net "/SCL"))
 (segment (start 80.1 73.6) (end 103.990991 73.6) (width 0.25) (layer "F.Cu") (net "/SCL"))
 (segment (start 79.75 73.405) (end 79.705 73.405) (width 0.25) (layer "F.Cu") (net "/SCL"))
 (segment (start 78.675 88.15) (end 90.077387 88.15) (width 0.25) (layer "F.Cu") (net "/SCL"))
 (segment (start 114.890991 55.3) (end 107.507236 55.3) (width 0.25) (layer "F.Cu") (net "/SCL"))
 (segment (start 118.125 58.534009) (end 114.890991 55.3) (width 0.25) (layer "F.Cu") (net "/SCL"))
 (segment (start 107.507236 55.3) (end 107.25 55.557236) (width 0.25) (layer "F.Cu") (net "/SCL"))
 (segment (start 103.990991 73.6) (end 118.125 59.465991) (width 0.25) (layer "F.Cu") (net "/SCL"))
 (segment (start 79.705 73.405) (end 79.6 73.3) (width 0.25) (layer "F.Cu") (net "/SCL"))
 (segment (start 118.575 59.652387) (end 118.575 58.347613) (width 0.25) (layer "F.Cu") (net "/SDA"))
 (segment (start 115.077387 54.85) (end 107.052556 54.85) (width 0.25) (layer "F.Cu") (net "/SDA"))
 (segment (start 101.012387 77.215) (end 118.575 59.652387) (width 0.25) (layer "F.Cu") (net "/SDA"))
 (segment (start 79.75 77.215) (end 101.012387 77.215) (width 0.25) (layer "F.Cu") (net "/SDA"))
 (segment (start 118.575 58.347613) (end 115.077387 54.85) (width 0.25) (layer "F.Cu") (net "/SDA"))
 (segment (start 106.5 55.402556) (end 106.5 56.007191) (width 0.25) (layer "F.Cu") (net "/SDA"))
 (segment (start 107.052556 54.85) (end 106.5 55.402556) (width 0.25) (layer "F.Cu") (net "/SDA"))
 (via (at 106.5 56.007191) (size 0.8) (drill 0.4) (layers "F.Cu" "B.Cu") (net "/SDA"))
 (via (at 79.75 77.215) (size 0.6) (drill 0.3) (layers "F.Cu" "B.Cu") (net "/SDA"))
 (segment (start 79.75 77.25) (end 79.8 77.3) (width 0.25) (layer "B.Cu") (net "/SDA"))
 (segment (start 79.75 77.215) (end 79.75 77.25) (width 0.25) (layer "B.Cu") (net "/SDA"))
 (segment (start 62.83 78.485) (end 70 85.655) (width 0.25) (layer "F.Cu") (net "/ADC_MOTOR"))
 (segment (start 44.42 98.5) (end 44.42 98.58) (width 0.25) (layer "F.Cu") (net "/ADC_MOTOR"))
 (segment (start 77.945 90.133884) (end 66.789442 101.289442) (width 0.25) (layer "F.Cu") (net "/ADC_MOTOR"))
 (segment (start 62.25 78.485) (end 62.83 78.485) (width 0.25) (layer "F.Cu") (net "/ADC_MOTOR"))
 (segment (start 44.42 98.58) (end 46.5 96.5) (width 0.25) (layer "F.Cu") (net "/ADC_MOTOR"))
 (segment (start 77.945 87.363604) (end 77.945 90.133884) (width 0.25) (layer "F.Cu") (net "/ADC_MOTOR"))
 (segment (start 76.236396 85.655) (end 77.945 87.363604) (width 0.25) (layer "F.Cu") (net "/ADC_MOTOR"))
 (segment (start 70 85.655) (end 76.236396 85.655) (width 0.25) (layer "F.Cu") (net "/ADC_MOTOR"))
 (segment (start 46.5 96.5) (end 58 96.5) (width 0.25) (layer "F.Cu") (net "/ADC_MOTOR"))
 (via (at 66.789442 101.289442) (size 0.6) (drill 0.3) (layers "F.Cu" "B.Cu") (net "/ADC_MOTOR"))
 (via (at 58.5 95.5) (size 0.6) (drill 0.3) (layers "F.Cu" "B.Cu") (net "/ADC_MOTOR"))
 (segment (start 66.789442 101.289442) (end 61 95.5) (width 0.25) (layer "B.Cu") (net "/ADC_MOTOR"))
 (segment (start 61 95.5) (end 58.5 95.5) (width 0.25) (layer "B.Cu") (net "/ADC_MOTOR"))
 (segment (start 36.034009 118.375) (end 39.635 118.375) (width 0.25) (layer "F.Cu") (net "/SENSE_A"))
 (segment (start 39.635 118.375) (end 41.43 116.58) (width 0.25) (layer "F.Cu") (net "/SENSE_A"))
 (segment (start 54.58 98.5) (end 54.58 106.152361) (width 0.25) (layer "F.Cu") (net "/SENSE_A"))
 (segment (start 54.58 98.5) (end 54.5 98.5) (width 0.25) (layer "F.Cu") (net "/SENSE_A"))
 (segment (start 40.107361 120.625) (end 36.034009 120.625) (width 0.25) (layer "F.Cu") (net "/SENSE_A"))
 (segment (start 35.375 119.034009) (end 36.034009 118.375) (width 0.25) (layer "F.Cu") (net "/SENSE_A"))
 (segment (start 35.375 119.965991) (end 35.375 119.034009) (width 0.25) (layer "F.Cu") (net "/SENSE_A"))
 (segment (start 54.5 98.5) (end 54.5 98.409009) (width 0.25) (layer "F.Cu") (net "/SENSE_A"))
 (segment (start 36.034009 120.625) (end 35.375 119.965991) (width 0.25) (layer "F.Cu") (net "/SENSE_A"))
 (segment (start 54.58 106.152361) (end 40.107361 120.625) (width 0.25) (layer "F.Cu") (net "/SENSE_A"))
 (segment (start 26.42056 115.078148) (end 28.421852 115.078148) (width 0.25) (layer "F.Cu") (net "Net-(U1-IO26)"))
 (segment (start 23.695 104.077613) (end 23.695 112.352588) (width 0.25) (layer "F.Cu") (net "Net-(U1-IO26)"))
 (segment (start 23.695 112.352588) (end 26.42056 115.078148) (width 0.25) (layer "F.Cu") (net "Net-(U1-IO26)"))
 (segment (start 44.207613 83.565) (end 23.695 104.077613) (width 0.25) (layer "F.Cu") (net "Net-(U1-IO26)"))
 (segment (start 62.25 83.565) (end 44.207613 83.565) (width 0.25) (layer "F.Cu") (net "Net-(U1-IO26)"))
 (via (at 28.421852 115.078148) (size 0.6) (drill 0.3) (layers "F.Cu" "B.Cu") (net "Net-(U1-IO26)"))
 (segment (start 28.421852 115.078148) (end 30 113.5) (width 0.25) (layer "B.Cu") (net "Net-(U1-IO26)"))
 (segment (start 30 113.5) (end 30 111.5) (width 0.25) (layer "B.Cu") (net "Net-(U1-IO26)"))
 (segment (start 26.235 112.007412) (end 30.807588 116.58) (width 0.25) (layer "F.Cu") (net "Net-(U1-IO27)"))
 (segment (start 43.574009 84.835) (end 24.375 104.034009) (width 0.25) (layer "F.Cu") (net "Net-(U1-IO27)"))
 (segment (start 24.375 109.132588) (end 26.235 110.992588) (width 0.25) (layer "F.Cu") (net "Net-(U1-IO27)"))
 (segment (start 24.375 104.034009) (end 24.375 109.132588) (width 0.25) (layer "F.Cu") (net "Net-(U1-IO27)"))
 (segment (start 26.235 110.992588) (end 26.235 112.007412) (width 0.25) (layer "F.Cu") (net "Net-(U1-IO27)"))
 (segment (start 62.25 84.835) (end 43.574009 84.835) (width 0.25) (layer "F.Cu") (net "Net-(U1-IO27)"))
 (segment (start 30.807588 116.58) (end 31.27 116.58) (width 0.25) (layer "F.Cu") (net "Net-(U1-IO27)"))
 (segment (start 77.495 89.7) (end 46.12 121.075) (width 0.25) (layer "F.Cu") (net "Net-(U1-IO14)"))
 (segment (start 28.73 118.73) (end 28.73 116.58) (width 0.25) (layer "F.Cu") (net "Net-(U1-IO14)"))
 (segment (start 46.12 121.075) (end 31.075 121.075) (width 0.25) (layer "F.Cu") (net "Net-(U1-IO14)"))
 (segment (start 76.05 86.105) (end 77.495 87.55) (width 0.25) (layer "F.Cu") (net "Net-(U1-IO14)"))
 (segment (start 77.495 87.55) (end 77.495 89.7) (width 0.25) (layer "F.Cu") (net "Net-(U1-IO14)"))
 (segment (start 31.075 121.075) (end 28.73 118.73) (width 0.25) (layer "F.Cu") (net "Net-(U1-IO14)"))
 (segment (start 62.25 86.105) (end 76.05 86.105) (width 0.25) (layer "F.Cu") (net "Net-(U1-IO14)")))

